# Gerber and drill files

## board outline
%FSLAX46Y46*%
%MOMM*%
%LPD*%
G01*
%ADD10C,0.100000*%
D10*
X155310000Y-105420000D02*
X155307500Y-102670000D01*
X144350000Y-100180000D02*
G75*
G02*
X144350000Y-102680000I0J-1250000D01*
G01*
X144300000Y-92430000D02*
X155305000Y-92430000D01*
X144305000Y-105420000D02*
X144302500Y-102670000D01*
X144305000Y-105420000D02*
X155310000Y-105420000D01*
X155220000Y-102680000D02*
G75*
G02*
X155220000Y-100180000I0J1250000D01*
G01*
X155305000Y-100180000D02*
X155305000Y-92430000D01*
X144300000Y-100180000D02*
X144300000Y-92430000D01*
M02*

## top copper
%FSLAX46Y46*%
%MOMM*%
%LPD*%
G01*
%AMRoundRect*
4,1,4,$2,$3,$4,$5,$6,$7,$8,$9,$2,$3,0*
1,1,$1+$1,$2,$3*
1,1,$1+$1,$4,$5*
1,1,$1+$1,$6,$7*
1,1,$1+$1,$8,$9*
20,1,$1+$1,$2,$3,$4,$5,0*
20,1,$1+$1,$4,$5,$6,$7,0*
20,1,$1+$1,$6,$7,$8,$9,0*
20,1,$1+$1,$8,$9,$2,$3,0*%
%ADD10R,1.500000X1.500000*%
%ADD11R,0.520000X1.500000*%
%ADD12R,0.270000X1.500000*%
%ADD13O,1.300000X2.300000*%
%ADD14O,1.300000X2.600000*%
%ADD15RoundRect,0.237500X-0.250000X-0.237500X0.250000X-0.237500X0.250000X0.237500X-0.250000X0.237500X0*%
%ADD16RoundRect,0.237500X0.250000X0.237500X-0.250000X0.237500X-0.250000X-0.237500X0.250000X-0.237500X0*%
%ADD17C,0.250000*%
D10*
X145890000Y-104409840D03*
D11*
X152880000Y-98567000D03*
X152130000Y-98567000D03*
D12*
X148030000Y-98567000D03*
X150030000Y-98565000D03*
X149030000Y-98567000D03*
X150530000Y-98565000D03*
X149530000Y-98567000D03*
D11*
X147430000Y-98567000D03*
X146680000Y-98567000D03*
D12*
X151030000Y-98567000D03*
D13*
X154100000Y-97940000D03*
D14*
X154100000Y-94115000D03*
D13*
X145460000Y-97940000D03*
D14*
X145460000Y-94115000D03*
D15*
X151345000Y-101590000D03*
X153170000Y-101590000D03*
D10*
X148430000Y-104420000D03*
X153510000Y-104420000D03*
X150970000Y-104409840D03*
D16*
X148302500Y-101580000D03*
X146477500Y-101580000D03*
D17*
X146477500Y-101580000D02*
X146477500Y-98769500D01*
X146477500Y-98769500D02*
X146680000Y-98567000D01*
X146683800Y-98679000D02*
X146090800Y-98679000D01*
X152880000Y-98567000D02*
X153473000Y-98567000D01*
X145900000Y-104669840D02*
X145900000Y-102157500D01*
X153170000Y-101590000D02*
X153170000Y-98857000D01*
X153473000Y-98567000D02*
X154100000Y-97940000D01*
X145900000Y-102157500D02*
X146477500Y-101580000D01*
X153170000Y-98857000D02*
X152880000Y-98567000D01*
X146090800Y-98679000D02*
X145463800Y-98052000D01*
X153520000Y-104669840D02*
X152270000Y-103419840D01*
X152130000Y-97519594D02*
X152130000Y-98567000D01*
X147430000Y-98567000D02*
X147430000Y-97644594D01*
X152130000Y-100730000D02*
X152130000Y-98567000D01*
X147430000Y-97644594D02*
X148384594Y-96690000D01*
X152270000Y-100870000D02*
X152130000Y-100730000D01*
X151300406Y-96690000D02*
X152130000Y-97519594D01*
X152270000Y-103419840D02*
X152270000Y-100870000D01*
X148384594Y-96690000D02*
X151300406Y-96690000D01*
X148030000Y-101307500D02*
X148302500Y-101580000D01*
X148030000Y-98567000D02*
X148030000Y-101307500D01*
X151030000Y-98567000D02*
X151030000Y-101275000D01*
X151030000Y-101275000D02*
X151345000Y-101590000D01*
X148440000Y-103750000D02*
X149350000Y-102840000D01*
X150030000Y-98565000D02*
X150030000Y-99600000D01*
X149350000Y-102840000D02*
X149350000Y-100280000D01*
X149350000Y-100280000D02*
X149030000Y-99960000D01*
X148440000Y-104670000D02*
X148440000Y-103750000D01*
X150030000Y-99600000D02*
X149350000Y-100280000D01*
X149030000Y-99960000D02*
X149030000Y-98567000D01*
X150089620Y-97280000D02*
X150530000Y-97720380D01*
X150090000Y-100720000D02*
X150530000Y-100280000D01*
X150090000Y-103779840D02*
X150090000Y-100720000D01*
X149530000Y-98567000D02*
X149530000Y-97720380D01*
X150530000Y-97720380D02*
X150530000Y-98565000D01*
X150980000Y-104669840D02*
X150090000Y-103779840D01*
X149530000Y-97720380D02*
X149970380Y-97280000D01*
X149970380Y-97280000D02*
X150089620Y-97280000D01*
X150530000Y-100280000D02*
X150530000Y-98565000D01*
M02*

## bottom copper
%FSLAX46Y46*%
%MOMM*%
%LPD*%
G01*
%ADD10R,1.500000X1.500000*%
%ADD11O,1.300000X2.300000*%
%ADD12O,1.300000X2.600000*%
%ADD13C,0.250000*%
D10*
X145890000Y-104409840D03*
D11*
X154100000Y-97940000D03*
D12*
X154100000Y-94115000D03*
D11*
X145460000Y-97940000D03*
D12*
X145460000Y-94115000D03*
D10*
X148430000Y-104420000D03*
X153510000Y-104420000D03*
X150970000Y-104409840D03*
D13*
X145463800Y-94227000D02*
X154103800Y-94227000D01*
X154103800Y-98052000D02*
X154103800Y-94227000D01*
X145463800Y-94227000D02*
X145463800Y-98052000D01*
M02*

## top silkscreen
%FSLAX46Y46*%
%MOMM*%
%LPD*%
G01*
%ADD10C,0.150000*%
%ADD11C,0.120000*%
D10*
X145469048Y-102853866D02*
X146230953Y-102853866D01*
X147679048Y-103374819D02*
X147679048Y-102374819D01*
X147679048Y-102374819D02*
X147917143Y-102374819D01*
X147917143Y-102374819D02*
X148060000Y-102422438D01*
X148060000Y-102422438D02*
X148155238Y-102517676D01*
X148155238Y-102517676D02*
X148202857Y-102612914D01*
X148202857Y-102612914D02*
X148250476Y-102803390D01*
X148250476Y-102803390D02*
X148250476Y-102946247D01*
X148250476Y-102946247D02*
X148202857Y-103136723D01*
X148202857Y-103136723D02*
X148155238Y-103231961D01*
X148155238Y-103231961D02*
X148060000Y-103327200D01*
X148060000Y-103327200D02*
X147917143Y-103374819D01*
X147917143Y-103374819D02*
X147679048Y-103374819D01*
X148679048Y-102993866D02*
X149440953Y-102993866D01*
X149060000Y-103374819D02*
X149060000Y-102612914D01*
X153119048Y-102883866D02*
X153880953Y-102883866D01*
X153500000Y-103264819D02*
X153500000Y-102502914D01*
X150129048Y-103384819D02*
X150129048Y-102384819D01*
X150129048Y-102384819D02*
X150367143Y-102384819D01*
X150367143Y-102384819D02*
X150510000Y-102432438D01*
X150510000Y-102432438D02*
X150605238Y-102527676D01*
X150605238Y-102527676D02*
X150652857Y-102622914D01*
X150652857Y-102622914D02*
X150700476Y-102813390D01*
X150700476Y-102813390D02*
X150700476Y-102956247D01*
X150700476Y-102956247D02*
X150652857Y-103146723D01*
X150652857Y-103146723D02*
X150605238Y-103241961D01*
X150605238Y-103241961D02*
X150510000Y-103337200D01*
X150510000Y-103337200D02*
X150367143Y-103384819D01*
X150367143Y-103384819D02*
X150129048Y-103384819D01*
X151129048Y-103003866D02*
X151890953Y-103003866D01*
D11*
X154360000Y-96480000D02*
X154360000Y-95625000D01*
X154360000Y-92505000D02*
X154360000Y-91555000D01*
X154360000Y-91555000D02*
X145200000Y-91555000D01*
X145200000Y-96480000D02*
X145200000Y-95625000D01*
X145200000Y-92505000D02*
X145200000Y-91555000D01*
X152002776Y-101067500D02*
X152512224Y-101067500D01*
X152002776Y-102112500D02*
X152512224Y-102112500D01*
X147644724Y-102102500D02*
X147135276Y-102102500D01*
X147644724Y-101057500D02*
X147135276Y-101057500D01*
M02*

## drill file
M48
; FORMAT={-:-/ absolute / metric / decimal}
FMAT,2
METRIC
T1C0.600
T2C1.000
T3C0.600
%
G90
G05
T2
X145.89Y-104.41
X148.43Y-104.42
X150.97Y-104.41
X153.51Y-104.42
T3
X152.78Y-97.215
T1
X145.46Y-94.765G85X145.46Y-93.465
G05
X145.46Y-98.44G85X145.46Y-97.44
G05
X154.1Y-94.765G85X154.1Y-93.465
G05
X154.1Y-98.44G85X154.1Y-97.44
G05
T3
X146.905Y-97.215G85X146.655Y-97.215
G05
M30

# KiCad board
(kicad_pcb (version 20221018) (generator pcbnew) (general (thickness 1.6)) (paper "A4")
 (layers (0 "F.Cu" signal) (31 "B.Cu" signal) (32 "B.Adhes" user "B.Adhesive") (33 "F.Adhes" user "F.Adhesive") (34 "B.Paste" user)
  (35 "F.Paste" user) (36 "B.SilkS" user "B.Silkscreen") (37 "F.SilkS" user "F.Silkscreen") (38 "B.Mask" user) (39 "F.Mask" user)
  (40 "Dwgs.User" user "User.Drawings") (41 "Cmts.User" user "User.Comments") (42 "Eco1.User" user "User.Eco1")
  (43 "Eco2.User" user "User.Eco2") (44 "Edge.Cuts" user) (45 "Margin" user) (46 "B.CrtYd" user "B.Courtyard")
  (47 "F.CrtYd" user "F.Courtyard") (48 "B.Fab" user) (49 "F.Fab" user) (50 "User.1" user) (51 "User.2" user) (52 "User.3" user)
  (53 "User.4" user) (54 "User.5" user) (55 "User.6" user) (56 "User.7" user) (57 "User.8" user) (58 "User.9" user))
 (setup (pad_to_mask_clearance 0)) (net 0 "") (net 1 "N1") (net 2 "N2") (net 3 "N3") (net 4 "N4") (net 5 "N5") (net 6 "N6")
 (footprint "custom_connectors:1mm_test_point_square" (layer "F.Cu") (at 145.89 104.42)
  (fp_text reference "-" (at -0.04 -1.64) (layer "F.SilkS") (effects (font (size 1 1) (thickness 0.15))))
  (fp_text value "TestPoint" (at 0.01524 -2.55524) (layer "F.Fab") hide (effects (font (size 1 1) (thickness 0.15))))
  (pad "1" thru_hole rect (at 0 -0.01016) (size 1.5 1.5) (drill 1) (layers "*.Cu" "*.Mask") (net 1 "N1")))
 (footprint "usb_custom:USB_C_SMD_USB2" (layer "F.Cu") (at 149.78 95.265 180)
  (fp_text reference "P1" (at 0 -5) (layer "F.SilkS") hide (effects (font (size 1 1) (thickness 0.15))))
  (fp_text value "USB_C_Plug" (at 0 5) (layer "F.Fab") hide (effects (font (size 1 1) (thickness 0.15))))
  (fp_line (start -4.58 -1.215) (end -4.58 -0.36) (stroke (width 0.12) (type solid)) (layer "F.SilkS"))
  (fp_line (start -4.58 2.76) (end -4.58 3.71) (stroke (width 0.12) (type solid)) (layer "F.SilkS"))
  (fp_line (start -4.58 3.71) (end 4.58 3.71) (stroke (width 0.12) (type solid)) (layer "F.SilkS"))
  (fp_line (start 4.58 -1.215) (end 4.58 -0.36) (stroke (width 0.12) (type solid)) (layer "F.SilkS"))
  (fp_line (start 4.58 2.76) (end 4.58 3.71) (stroke (width 0.12) (type solid)) (layer "F.SilkS"))
  (pad "" np_thru_hole circle (at -3 -1.95 180) (size 0.6 0.6) (drill 0.6) (layers "F&B.Cu" "*.Mask"))
  (pad "" np_thru_hole oval (at 3 -1.95 180) (size 0.85 0.6) (drill oval 0.85 0.6) (layers "F&B.Cu" "*.Mask"))
  (pad "A1" smd rect (at -3.1 -3.302 180) (size 0.52 1.5) (layers "F.Cu" "F.Paste" "F.Mask") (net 1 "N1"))
  (pad "A4" smd rect (at -2.35 -3.302 180) (size 0.52 1.5) (layers "F.Cu" "F.Paste" "F.Mask") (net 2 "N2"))
  (pad "A5" smd rect (at 1.75 -3.302 180) (size 0.27 1.5) (layers "F.Cu" "F.Paste" "F.Mask") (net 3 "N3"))
  (pad "A6" smd rect (at -0.25 -3.3 180) (size 0.27 1.5) (layers "F.Cu" "F.Paste" "F.Mask") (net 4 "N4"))
  (pad "A6" smd rect (at 0.75 -3.302 180) (size 0.27 1.5) (layers "F.Cu" "F.Paste" "F.Mask") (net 4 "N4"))
  (pad "A7" smd rect (at -0.75 -3.3 180) (size 0.27 1.5) (layers "F.Cu" "F.Paste" "F.Mask") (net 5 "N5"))
  (pad "A7" smd rect (at 0.25 -3.302 180) (size 0.27 1.5) (layers "F.Cu" "F.Paste" "F.Mask") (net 5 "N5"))
  (pad "A9" smd rect (at 2.35 -3.302 180) (size 0.52 1.5) (layers "F.Cu" "F.Paste" "F.Mask") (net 2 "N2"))
  (pad "A12" smd rect (at 3.1 -3.302 180) (size 0.52 1.5) (layers "F.Cu" "F.Paste" "F.Mask") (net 1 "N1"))
  (pad "B5" smd rect (at -1.25 -3.302 180) (size 0.27 1.5) (layers "F.Cu" "F.Paste" "F.Mask") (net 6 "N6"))
  (pad "S1" thru_hole oval (at -4.32 -2.675 180) (size 1.3 2.3) (drill oval 0.6 1.6) (layers "*.Cu" "*.Mask") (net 1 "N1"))
  (pad "S1" thru_hole oval (at -4.32 1.15 180) (size 1.3 2.6) (drill oval 0.6 1.9) (layers "*.Cu" "*.Mask") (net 1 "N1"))
  (pad "S1" thru_hole oval (at 4.32 -2.675 180) (size 1.3 2.3) (drill oval 0.6 1.6) (layers "*.Cu" "*.Mask") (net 1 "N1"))
  (pad "S1" thru_hole oval (at 4.32 1.15 180) (size 1.3 2.6) (drill oval 0.6 1.9) (layers "*.Cu" "*.Mask") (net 1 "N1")))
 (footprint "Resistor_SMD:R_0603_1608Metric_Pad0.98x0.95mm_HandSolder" (layer "F.Cu") (at 152.2575 101.59)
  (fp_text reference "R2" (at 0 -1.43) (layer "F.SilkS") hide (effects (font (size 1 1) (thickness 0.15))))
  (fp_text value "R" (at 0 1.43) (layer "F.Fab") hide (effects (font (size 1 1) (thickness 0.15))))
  (fp_line (start -0.254724 -0.5225) (end 0.254724 -0.5225) (stroke (width 0.12) (type solid)) (layer "F.SilkS"))
  (fp_line (start -0.254724 0.5225) (end 0.254724 0.5225) (stroke (width 0.12) (type solid)) (layer "F.SilkS"))
  (pad "1" smd roundrect (at -0.9125 0) (size 0.975 0.95) (layers "F.Cu" "F.Paste" "F.Mask") (roundrect_rratio 0.25) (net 6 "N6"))
  (pad "2" smd roundrect (at 0.9125 0) (size 0.975 0.95) (layers "F.Cu" "F.Paste" "F.Mask") (roundrect_rratio 0.25) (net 1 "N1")))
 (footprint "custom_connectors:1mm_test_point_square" (layer "F.Cu") (at 148.43 104.43016)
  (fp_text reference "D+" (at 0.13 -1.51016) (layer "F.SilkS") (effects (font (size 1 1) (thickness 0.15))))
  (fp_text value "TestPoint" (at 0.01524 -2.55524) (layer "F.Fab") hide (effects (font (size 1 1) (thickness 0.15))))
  (pad "1" thru_hole rect (at 0 -0.01016) (size 1.5 1.5) (drill 1) (layers "*.Cu" "*.Mask") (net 4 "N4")))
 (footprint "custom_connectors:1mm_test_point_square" (layer "F.Cu") (at 153.51 104.43016)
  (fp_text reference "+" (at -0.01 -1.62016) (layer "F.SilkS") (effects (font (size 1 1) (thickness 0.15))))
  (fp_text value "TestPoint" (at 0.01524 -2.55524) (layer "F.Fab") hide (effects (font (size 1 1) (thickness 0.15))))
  (pad "1" thru_hole rect (at 0 -0.01016) (size 1.5 1.5) (drill 1) (layers "*.Cu" "*.Mask") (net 2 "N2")))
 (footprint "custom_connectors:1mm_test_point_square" (layer "F.Cu") (at 150.97 104.42)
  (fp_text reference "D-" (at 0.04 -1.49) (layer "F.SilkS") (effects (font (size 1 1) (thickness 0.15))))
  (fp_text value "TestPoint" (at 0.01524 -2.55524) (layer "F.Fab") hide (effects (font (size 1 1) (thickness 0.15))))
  (pad "1" thru_hole rect (at 0 -0.01016) (size 1.5 1.5) (drill 1) (layers "*.Cu" "*.Mask") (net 5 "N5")))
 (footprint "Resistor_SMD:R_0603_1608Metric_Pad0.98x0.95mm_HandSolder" (layer "F.Cu") (at 147.39 101.58 180)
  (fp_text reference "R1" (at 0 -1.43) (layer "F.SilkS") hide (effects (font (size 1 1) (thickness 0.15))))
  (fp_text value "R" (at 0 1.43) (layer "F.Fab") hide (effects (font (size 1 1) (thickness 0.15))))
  (fp_line (start -0.254724 -0.5225) (end 0.254724 -0.5225) (stroke (width 0.12) (type solid)) (layer "F.SilkS"))
  (fp_line (start -0.254724 0.5225) (end 0.254724 0.5225) (stroke (width 0.12) (type solid)) (layer "F.SilkS"))
  (pad "1" smd roundrect (at -0.9125 0 180) (size 0.975 0.95) (layers "F.Cu" "F.Paste" "F.Mask") (roundrect_rratio 0.25) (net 3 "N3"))
  (pad "2" smd roundrect (at 0.9125 0 180) (size 0.975 0.95) (layers "F.Cu" "F.Paste" "F.Mask") (roundrect_rratio 0.25) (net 1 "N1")))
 (gr_line (start 155.31 105.42) (end 155.3075 102.67) (stroke (width 0.1) (type default)) (layer "Edge.Cuts"))
 (gr_arc (start 144.35 100.18) (mid 145.6 101.43) (end 144.35 102.68) (stroke (width 0.1) (type default)) (layer "Edge.Cuts"))
 (gr_line (start 144.3 92.43) (end 155.305 92.43) (stroke (width 0.1) (type default)) (layer "Edge.Cuts"))
 (gr_line (start 144.305 105.42) (end 144.3025 102.67) (stroke (width 0.1) (type default)) (layer "Edge.Cuts"))
 (gr_line (start 144.305 105.42) (end 155.31 105.42) (stroke (width 0.1) (type default)) (layer "Edge.Cuts"))
 (gr_arc (start 155.22 102.68) (mid 153.97 101.43) (end 155.22 100.18) (stroke (width 0.1) (type default)) (layer "Edge.Cuts"))
 (gr_line (start 155.305 100.18) (end 155.305 92.43) (stroke (width 0.1) (type default)) (layer "Edge.Cuts"))
 (gr_line (start 144.3 100.18) (end 144.3 92.43) (stroke (width 0.1) (type default)) (layer "Edge.Cuts"))
 (segment (start 146.4775 101.58) (end 146.4775 98.7695) (width 0.25) (layer "F.Cu") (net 1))
 (segment (start 146.4775 98.7695) (end 146.68 98.567) (width 0.25) (layer "F.Cu") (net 1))
 (segment (start 146.6838 98.679) (end 146.0908 98.679) (width 0.25) (layer "F.Cu") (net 1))
 (segment (start 152.88 98.567) (end 153.473 98.567) (width 0.25) (layer "F.Cu") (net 1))
 (segment (start 145.9 104.66984) (end 145.9 102.1575) (width 0.25) (layer "F.Cu") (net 1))
 (segment (start 153.17 101.59) (end 153.17 98.857) (width 0.25) (layer "F.Cu") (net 1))
 (segment (start 153.473 98.567) (end 154.1 97.94) (width 0.25) (layer "F.Cu") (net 1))
 (segment (start 145.9 102.1575) (end 146.4775 101.58) (width 0.25) (layer "F.Cu") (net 1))
 (segment (start 153.17 98.857) (end 152.88 98.567) (width 0.25) (layer "F.Cu") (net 1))
 (segment (start 146.0908 98.679) (end 145.4638 98.052) (width 0.25) (layer "F.Cu") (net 1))
 (segment (start 145.4638 94.227) (end 154.1038 94.227) (width 0.25) (layer "B.Cu") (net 1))
 (segment (start 154.1038 98.052) (end 154.1038 94.227) (width 0.25) (layer "B.Cu") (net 1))
 (segment (start 145.4638 94.227) (end 145.4638 98.052) (width 0.25) (layer "B.Cu") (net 1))
 (segment (start 153.52 104.66984) (end 152.27 103.41984) (width 0.25) (layer "F.Cu") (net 2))
 (segment (start 152.13 97.519594) (end 152.13 98.567) (width 0.25) (layer "F.Cu") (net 2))
 (segment (start 147.43 98.567) (end 147.43 97.644594) (width 0.25) (layer "F.Cu") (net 2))
 (segment (start 152.13 100.73) (end 152.13 98.567) (width 0.25) (layer "F.Cu") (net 2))
 (segment (start 147.43 97.644594) (end 148.384594 96.69) (width 0.25) (layer "F.Cu") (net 2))
 (segment (start 152.27 100.87) (end 152.13 100.73) (width 0.25) (layer "F.Cu") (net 2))
 (segment (start 151.300406 96.69) (end 152.13 97.519594) (width 0.25) (layer "F.Cu") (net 2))
 (segment (start 152.27 103.41984) (end 152.27 100.87) (width 0.25) (layer "F.Cu") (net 2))
 (segment (start 148.384594 96.69) (end 151.300406 96.69) (width 0.25) (layer "F.Cu") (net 2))
 (segment (start 148.03 101.3075) (end 148.3025 101.58) (width 0.25) (layer "F.Cu") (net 3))
 (segment (start 148.03 98.567) (end 148.03 101.3075) (width 0.25) (layer "F.Cu") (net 3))
 (segment (start 151.03 98.567) (end 151.03 101.275) (width 0.25) (layer "F.Cu") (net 6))
 (segment (start 151.03 101.275) (end 151.345 101.59) (width 0.25) (layer "F.Cu") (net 6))
 (segment (start 148.44 103.75) (end 149.35 102.84) (width 0.25) (layer "F.Cu") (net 4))
 (segment (start 150.03 98.565) (end 150.03 99.6) (width 0.25) (layer "F.Cu") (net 4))
 (segment (start 149.35 102.84) (end 149.35 100.28) (width 0.25) (layer "F.Cu") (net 4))
 (segment (start 149.35 100.28) (end 149.03 99.96) (width 0.25) (layer "F.Cu") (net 4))
 (segment (start 148.44 104.67) (end 148.44 103.75) (width 0.25) (layer "F.Cu") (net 4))
 (segment (start 150.03 99.6) (end 149.35 100.28) (width 0.25) (layer "F.Cu") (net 4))
 (segment (start 149.03 99.96) (end 149.03 98.567) (width 0.25) (layer "F.Cu") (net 4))
 (segment (start 150.08962 97.28) (end 150.53 97.72038) (width 0.25) (layer "F.Cu") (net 5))
 (segment (start 150.09 100.72) (end 150.53 100.28) (width 0.25) (layer "F.Cu") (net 5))
 (segment (start 150.09 103.77984) (end 150.09 100.72) (width 0.25) (layer "F.Cu") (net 5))
 (segment (start 149.53 98.567) (end 149.53 97.72038) (width 0.25) (layer "F.Cu") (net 5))
 (segment (start 150.53 97.72038) (end 150.53 98.565) (width 0.25) (layer "F.Cu") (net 5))
 (segment (start 150.98 104.66984) (end 150.09 103.77984) (width 0.25) (layer "F.Cu") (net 5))
 (segment (start 149.53 97.72038) (end 149.97038 97.28) (width 0.25) (layer "F.Cu") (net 5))
 (segment (start 149.97038 97.28) (end 150.08962 97.28) (width 0.25) (layer "F.Cu") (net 5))
 (segment (start 150.53 100.28) (end 150.53 98.565) (width 0.25) (layer "F.Cu") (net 5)))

